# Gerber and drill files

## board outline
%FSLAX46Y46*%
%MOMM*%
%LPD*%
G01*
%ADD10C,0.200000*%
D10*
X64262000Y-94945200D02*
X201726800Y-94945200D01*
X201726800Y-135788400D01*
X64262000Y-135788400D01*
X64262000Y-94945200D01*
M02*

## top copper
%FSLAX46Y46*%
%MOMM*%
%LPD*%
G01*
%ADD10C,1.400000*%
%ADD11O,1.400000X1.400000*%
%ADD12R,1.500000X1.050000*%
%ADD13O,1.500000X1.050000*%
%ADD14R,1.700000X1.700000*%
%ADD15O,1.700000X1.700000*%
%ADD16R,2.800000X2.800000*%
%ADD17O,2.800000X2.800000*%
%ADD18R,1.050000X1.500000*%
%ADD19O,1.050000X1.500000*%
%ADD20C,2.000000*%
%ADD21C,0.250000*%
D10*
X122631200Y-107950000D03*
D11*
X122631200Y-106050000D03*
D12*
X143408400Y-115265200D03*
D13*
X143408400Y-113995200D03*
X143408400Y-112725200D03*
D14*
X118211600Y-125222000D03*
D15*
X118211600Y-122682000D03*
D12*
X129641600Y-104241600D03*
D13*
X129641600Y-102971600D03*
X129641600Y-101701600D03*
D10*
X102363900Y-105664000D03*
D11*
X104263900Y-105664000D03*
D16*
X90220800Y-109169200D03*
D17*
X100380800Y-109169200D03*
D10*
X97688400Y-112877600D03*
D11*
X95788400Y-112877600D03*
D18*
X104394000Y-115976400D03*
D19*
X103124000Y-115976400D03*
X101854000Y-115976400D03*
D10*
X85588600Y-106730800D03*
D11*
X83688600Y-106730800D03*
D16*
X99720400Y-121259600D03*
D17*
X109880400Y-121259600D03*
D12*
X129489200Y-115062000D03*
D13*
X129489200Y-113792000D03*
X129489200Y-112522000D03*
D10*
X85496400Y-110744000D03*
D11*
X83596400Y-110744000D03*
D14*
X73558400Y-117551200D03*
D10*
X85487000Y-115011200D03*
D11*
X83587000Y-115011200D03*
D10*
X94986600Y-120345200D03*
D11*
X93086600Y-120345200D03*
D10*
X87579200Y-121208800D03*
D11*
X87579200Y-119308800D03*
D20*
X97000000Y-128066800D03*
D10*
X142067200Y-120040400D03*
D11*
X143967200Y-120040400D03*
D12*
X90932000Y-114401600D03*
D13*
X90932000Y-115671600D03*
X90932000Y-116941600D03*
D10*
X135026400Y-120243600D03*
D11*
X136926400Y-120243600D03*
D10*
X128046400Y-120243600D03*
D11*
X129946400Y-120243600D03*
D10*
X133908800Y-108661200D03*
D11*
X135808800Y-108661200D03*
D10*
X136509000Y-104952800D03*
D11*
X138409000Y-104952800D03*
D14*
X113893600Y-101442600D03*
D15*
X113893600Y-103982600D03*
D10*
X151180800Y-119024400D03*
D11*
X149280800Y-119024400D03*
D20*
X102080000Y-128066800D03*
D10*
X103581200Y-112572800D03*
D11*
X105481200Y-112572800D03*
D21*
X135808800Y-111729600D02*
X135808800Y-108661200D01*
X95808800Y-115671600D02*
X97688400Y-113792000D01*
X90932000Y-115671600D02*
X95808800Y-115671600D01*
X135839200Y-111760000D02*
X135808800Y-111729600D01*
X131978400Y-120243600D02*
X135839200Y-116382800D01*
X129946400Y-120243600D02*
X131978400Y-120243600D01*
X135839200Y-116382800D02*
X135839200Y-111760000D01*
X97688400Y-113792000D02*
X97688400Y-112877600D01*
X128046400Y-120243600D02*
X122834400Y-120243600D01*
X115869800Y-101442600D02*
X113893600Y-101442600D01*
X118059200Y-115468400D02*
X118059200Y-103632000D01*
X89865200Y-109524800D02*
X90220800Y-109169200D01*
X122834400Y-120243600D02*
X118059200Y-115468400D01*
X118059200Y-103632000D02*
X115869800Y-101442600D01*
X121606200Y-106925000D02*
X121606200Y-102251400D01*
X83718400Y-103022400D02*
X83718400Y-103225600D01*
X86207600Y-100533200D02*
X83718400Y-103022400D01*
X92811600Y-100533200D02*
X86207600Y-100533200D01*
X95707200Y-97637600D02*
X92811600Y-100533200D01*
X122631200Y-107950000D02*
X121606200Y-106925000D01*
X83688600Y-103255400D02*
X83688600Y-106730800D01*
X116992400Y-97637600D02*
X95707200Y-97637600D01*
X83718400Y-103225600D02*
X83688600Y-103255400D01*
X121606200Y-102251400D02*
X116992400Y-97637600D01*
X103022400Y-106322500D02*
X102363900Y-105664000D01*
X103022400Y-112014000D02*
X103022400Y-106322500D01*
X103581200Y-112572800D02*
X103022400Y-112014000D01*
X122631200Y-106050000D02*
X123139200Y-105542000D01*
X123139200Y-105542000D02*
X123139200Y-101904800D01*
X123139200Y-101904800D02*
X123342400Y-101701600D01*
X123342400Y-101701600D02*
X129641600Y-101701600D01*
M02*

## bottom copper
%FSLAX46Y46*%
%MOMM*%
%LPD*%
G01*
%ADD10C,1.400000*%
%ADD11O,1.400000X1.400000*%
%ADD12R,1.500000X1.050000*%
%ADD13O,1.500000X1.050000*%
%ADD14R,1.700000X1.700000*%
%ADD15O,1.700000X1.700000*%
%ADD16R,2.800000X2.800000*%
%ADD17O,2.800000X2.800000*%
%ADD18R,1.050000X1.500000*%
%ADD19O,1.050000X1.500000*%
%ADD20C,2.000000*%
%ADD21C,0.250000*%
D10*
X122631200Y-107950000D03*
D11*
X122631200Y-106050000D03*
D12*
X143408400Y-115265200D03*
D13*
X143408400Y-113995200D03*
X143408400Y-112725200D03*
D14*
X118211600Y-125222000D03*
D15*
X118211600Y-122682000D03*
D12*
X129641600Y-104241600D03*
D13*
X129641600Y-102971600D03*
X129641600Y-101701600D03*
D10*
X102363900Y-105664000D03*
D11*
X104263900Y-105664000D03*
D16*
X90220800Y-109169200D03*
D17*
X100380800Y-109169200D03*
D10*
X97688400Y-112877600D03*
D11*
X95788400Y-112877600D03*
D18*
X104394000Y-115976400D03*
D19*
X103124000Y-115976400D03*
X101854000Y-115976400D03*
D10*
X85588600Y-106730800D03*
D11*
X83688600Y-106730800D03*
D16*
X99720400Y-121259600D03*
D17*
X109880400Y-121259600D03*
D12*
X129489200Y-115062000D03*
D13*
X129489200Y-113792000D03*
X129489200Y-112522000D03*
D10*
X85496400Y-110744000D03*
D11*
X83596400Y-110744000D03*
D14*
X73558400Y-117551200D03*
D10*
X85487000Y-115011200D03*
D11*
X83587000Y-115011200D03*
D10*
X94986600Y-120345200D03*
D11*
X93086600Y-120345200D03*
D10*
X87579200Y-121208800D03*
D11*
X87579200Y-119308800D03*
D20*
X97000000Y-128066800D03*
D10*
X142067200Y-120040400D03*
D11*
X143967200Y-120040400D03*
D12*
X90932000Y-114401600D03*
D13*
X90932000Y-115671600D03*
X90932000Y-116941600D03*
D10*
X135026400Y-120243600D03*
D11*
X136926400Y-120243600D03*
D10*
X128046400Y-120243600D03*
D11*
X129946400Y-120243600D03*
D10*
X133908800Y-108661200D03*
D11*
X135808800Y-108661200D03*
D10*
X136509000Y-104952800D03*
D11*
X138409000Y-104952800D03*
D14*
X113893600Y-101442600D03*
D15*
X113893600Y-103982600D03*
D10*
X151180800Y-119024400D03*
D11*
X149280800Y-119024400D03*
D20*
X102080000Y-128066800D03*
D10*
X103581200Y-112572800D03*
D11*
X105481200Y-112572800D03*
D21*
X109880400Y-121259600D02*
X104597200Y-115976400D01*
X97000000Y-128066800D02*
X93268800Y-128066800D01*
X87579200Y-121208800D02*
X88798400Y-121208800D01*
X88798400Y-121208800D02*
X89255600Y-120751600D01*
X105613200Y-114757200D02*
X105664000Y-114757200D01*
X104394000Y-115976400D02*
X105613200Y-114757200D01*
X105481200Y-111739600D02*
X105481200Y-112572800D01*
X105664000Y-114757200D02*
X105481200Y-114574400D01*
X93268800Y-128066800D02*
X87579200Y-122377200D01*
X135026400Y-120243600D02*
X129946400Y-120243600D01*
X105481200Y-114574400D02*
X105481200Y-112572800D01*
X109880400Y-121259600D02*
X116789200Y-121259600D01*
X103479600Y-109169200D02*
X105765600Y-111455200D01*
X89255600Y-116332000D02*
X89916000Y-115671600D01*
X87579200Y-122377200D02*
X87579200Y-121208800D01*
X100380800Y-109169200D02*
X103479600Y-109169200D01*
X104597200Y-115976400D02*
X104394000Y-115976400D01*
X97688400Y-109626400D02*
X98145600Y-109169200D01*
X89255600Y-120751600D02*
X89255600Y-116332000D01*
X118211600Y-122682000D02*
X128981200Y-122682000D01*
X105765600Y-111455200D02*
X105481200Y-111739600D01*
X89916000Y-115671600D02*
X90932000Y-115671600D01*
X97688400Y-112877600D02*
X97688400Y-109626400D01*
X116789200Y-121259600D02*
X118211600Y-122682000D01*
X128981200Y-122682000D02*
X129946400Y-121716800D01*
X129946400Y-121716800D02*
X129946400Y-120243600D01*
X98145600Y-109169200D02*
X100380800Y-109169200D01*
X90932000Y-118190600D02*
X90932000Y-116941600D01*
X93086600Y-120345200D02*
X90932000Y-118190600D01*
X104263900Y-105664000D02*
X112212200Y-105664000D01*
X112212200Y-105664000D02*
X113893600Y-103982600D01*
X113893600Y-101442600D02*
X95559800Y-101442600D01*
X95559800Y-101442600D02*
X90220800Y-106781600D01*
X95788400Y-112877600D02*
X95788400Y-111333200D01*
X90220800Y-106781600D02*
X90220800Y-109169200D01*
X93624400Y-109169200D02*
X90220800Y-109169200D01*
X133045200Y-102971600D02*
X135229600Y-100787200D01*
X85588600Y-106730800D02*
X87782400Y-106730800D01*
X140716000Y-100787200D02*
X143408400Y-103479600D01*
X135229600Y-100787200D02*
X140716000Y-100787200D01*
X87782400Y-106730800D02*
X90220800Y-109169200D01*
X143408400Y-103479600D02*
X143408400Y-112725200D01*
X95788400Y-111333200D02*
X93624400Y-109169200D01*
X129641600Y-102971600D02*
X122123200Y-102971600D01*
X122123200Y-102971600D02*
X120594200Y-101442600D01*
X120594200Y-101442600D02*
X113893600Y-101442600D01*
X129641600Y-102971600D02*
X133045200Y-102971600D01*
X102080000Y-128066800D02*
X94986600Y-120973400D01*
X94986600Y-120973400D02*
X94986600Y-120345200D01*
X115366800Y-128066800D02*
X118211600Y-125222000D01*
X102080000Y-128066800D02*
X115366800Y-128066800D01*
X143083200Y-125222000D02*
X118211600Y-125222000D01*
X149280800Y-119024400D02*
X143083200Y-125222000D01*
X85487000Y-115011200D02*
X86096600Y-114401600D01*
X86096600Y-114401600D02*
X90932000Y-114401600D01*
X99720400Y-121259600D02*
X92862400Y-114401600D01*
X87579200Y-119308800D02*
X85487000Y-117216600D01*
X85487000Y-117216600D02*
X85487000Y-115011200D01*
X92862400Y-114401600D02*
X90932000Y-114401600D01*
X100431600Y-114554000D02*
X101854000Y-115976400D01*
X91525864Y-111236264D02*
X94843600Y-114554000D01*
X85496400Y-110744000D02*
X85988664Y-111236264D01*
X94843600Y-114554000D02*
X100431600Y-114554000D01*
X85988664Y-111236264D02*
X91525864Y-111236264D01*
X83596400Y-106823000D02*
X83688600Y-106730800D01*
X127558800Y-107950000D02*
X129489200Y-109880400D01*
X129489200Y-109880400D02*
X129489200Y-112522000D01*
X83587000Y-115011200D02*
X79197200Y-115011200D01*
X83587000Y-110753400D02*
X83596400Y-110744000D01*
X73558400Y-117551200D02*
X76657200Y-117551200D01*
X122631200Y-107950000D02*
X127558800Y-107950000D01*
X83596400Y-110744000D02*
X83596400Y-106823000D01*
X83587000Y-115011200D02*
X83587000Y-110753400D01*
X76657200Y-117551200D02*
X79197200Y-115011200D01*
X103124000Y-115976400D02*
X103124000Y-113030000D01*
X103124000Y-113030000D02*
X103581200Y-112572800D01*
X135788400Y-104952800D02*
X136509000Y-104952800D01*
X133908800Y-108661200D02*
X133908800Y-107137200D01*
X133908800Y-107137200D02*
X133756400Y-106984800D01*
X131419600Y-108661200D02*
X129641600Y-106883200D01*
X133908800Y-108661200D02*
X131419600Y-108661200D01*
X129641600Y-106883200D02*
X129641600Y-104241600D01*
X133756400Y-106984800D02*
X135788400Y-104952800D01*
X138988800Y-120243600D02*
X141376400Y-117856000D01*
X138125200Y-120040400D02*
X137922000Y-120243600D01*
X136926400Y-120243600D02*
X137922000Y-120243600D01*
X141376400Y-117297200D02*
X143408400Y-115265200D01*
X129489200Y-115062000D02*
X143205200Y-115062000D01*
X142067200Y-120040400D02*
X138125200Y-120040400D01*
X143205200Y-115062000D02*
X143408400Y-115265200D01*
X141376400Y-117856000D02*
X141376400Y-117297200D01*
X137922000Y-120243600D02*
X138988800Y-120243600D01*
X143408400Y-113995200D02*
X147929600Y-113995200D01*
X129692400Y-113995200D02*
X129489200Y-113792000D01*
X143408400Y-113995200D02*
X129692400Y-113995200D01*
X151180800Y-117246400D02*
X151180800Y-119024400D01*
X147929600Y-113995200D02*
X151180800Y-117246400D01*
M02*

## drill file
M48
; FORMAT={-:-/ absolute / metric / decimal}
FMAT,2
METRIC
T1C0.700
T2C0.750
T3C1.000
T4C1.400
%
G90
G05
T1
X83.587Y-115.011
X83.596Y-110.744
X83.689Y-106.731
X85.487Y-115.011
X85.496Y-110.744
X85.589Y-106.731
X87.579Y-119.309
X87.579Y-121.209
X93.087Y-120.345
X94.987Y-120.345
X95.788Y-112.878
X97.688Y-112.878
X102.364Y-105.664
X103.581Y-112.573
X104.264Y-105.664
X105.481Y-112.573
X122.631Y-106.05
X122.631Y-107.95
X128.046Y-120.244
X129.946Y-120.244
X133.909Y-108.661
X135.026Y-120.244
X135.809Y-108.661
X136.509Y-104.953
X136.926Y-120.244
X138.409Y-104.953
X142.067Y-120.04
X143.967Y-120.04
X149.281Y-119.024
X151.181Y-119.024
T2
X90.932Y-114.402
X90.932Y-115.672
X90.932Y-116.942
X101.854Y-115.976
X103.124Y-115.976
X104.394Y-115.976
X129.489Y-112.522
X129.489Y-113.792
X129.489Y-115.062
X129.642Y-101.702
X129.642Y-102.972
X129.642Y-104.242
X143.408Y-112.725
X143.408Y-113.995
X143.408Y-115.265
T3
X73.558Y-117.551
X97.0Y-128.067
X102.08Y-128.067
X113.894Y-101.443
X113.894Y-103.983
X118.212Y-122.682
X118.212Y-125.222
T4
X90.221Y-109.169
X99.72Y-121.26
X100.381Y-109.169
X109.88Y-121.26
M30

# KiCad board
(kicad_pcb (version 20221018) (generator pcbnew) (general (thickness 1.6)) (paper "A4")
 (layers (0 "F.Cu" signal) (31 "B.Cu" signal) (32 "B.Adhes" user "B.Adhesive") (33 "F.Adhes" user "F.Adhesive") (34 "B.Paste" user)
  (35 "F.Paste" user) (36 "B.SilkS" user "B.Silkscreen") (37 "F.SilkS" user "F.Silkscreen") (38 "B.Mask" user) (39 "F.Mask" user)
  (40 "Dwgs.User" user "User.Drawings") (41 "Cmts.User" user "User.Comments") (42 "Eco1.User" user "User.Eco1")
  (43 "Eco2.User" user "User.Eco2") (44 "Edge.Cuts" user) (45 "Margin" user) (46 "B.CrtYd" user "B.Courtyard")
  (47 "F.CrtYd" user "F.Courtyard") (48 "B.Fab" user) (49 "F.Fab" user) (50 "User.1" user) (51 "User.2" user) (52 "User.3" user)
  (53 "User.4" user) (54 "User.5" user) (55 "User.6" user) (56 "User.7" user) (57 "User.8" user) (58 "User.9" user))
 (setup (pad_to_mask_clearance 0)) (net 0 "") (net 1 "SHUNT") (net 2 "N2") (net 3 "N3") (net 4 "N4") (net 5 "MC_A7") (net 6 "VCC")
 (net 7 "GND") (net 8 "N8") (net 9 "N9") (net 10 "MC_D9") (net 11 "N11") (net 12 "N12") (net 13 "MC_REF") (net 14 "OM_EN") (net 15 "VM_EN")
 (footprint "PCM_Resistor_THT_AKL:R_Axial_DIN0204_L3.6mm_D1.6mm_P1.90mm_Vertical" (layer "F.Cu") (at 122.6312 107.95 90)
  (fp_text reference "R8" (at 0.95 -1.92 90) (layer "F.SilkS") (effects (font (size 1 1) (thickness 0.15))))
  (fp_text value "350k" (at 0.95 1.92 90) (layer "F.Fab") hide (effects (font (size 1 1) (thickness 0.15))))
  (pad "1" thru_hole circle (at 0 0 90) (size 1.4 1.4) (drill 0.7) (layers "*.Cu" "*.Mask") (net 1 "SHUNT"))
  (pad "2" thru_hole oval (at 1.9 0 90) (size 1.4 1.4) (drill 0.7) (layers "*.Cu" "*.Mask") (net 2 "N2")))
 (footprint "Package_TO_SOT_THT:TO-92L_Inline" (layer "F.Cu") (at 143.4084 115.2652 90)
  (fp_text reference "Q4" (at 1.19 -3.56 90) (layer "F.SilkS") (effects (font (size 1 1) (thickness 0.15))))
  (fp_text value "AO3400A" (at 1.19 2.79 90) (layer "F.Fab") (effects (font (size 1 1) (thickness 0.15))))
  (pad "1" thru_hole rect (at 0 0 90) (size 1.05 1.5) (drill 0.75) (layers "*.Cu" "*.Mask") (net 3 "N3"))
  (pad "2" thru_hole oval (at 1.27 0 90) (size 1.05 1.5) (drill 0.75) (layers "*.Cu" "*.Mask") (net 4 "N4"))
  (pad "3" thru_hole oval (at 2.54 0 90) (size 1.05 1.5) (drill 0.75) (layers "*.Cu" "*.Mask") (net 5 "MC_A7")))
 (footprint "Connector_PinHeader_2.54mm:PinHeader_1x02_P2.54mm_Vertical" (layer "F.Cu") (at 118.2116 125.222 180)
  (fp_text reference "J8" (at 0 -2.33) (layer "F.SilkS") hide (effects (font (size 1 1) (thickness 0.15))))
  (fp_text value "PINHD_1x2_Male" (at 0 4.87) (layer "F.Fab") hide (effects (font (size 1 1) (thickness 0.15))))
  (pad "1" thru_hole rect (at 0 0 180) (size 1.7 1.7) (drill 1) (layers "*.Cu" "*.Mask") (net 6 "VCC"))
  (pad "2" thru_hole oval (at 0 2.54 180) (size 1.7 1.7) (drill 1) (layers "*.Cu" "*.Mask") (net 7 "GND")))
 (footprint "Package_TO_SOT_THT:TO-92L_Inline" (layer "F.Cu") (at 129.6416 104.2416 90)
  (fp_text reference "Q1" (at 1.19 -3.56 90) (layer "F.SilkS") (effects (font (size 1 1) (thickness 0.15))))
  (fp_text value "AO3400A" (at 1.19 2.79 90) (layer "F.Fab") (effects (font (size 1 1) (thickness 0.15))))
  (pad "1" thru_hole rect (at 0 0 90) (size 1.05 1.5) (drill 0.75) (layers "*.Cu" "*.Mask") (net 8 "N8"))
  (pad "2" thru_hole oval (at 1.27 0 90) (size 1.05 1.5) (drill 0.75) (layers "*.Cu" "*.Mask") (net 5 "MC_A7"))
  (pad "3" thru_hole oval (at 2.54 0 90) (size 1.05 1.5) (drill 0.75) (layers "*.Cu" "*.Mask") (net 2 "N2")))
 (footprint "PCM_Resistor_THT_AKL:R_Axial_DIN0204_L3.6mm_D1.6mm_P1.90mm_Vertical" (layer "F.Cu") (at 102.3639 105.664)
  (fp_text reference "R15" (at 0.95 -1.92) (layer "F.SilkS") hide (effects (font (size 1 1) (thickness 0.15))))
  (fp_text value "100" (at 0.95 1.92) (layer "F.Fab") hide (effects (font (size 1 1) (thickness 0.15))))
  (pad "1" thru_hole circle (at 0 0) (size 1.4 1.4) (drill 0.7) (layers "*.Cu" "*.Mask") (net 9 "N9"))
  (pad "2" thru_hole oval (at 1.9 0) (size 1.4 1.4) (drill 0.7) (layers "*.Cu" "*.Mask") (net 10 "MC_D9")))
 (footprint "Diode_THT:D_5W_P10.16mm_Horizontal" (layer "F.Cu") (at 90.2208 109.1692)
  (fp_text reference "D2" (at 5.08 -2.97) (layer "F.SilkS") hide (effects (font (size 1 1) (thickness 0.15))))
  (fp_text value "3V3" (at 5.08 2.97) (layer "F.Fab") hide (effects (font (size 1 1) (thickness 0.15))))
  (pad "1" thru_hole rect (at 0 0) (size 2.8 2.8) (drill 1.4) (layers "*.Cu" "*.Mask") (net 5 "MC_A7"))
  (pad "2" thru_hole oval (at 10.16 0) (size 2.8 2.8) (drill 1.4) (layers "*.Cu" "*.Mask") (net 7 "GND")))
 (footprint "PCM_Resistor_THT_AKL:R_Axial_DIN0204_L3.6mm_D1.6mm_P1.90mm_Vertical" (layer "F.Cu") (at 97.6884 112.8776 180)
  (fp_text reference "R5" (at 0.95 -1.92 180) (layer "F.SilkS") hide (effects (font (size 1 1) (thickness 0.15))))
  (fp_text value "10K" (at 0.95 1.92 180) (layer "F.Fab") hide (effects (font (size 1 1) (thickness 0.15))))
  (pad "1" thru_hole circle (at 0 0 180) (size 1.4 1.4) (drill 0.7) (layers "*.Cu" "*.Mask") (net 7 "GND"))
  (pad "2" thru_hole oval (at 1.9 0 180) (size 1.4 1.4) (drill 0.7) (layers "*.Cu" "*.Mask") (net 5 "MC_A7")))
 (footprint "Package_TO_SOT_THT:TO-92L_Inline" (layer "F.Cu") (at 104.394 115.9764 180)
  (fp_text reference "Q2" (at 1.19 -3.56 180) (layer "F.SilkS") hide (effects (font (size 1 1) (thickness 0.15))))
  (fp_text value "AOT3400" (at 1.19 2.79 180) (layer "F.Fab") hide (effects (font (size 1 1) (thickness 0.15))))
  (pad "1" thru_hole rect (at 0 0 180) (size 1.05 1.5) (drill 0.75) (layers "*.Cu" "*.Mask") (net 7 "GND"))
  (pad "2" thru_hole oval (at 1.27 0 180) (size 1.05 1.5) (drill 0.75) (layers "*.Cu" "*.Mask") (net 9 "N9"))
  (pad "3" thru_hole oval (at 2.54 0 180) (size 1.05 1.5) (drill 0.75) (layers "*.Cu" "*.Mask") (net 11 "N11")))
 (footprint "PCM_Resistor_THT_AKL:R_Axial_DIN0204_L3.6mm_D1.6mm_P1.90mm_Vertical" (layer "F.Cu") (at 85.5886 106.7308 180)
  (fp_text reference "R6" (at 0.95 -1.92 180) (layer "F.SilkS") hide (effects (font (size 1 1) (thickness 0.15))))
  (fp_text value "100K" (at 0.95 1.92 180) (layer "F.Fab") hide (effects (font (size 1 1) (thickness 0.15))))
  (pad "1" thru_hole circle (at 0 0 180) (size 1.4 1.4) (drill 0.7) (layers "*.Cu" "*.Mask") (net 5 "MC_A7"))
  (pad "2" thru_hole oval (at 1.9 0 180) (size 1.4 1.4) (drill 0.7) (layers "*.Cu" "*.Mask") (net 1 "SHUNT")))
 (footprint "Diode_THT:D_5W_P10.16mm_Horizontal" (layer "F.Cu") (at 99.7204 121.2596)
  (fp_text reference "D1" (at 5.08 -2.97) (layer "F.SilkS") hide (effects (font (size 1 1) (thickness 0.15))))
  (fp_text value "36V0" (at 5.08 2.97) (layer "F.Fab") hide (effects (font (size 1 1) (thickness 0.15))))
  (pad "1" thru_hole rect (at 0 0) (size 2.8 2.8) (drill 1.4) (layers "*.Cu" "*.Mask") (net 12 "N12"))
  (pad "2" thru_hole oval (at 10.16 0) (size 2.8 2.8) (drill 1.4) (layers "*.Cu" "*.Mask") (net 7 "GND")))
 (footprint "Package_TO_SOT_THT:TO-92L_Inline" (layer "F.Cu") (at 129.4892 115.062 90)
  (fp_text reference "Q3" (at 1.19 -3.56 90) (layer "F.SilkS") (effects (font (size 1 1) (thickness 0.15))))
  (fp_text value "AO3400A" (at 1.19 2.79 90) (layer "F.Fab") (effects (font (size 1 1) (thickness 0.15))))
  (pad "1" thru_hole rect (at 0 0 90) (size 1.05 1.5) (drill 0.75) (layers "*.Cu" "*.Mask") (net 3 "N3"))
  (pad "2" thru_hole oval (at 1.27 0 90) (size 1.05 1.5) (drill 0.75) (layers "*.Cu" "*.Mask") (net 4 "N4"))
  (pad "3" thru_hole oval (at 2.54 0 90) (size 1.05 1.5) (drill 0.75) (layers "*.Cu" "*.Mask") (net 1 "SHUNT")))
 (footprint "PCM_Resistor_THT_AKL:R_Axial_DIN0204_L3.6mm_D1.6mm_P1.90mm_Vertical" (layer "F.Cu") (at 85.4964 110.744 180)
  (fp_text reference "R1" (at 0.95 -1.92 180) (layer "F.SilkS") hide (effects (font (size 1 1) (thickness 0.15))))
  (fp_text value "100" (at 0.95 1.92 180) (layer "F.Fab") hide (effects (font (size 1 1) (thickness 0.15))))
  (pad "1" thru_hole circle (at 0 0 180) (size 1.4 1.4) (drill 0.7) (layers "*.Cu" "*.Mask") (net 11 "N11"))
  (pad "2" thru_hole oval (at 1.9 0 180) (size 1.4 1.4) (drill 0.7) (layers "*.Cu" "*.Mask") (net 1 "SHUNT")))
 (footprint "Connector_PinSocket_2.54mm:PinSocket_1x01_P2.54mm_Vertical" (layer "F.Cu") (at 73.5584 117.5512)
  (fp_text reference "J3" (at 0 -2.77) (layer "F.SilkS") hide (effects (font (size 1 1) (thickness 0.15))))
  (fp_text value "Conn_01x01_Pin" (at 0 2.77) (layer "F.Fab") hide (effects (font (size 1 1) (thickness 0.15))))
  (pad "1" thru_hole rect (at 0 0) (size 1.7 1.7) (drill 1) (layers "*.Cu" "*.Mask") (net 1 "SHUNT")))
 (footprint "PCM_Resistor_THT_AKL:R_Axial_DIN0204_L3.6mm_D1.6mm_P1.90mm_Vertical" (layer "F.Cu") (at 85.487 115.0112 180)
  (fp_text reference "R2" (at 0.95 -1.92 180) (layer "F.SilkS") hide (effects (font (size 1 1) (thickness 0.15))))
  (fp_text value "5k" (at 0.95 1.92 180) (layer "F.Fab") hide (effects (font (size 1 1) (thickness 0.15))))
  (pad "1" thru_hole circle (at 0 0 180) (size 1.4 1.4) (drill 0.7) (layers "*.Cu" "*.Mask") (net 12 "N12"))
  (pad "2" thru_hole oval (at 1.9 0 180) (size 1.4 1.4) (drill 0.7) (layers "*.Cu" "*.Mask") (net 1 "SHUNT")))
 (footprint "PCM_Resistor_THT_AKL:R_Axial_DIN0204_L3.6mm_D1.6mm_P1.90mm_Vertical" (layer "F.Cu") (at 94.9866 120.3452 180)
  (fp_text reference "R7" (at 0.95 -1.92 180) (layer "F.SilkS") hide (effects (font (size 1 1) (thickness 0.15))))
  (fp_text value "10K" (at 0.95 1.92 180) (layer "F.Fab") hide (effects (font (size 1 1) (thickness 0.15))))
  (pad "1" thru_hole circle (at 0 0 180) (size 1.4 1.4) (drill 0.7) (layers "*.Cu" "*.Mask") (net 6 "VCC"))
  (pad "2" thru_hole oval (at 1.9 0 180) (size 1.4 1.4) (drill 0.7) (layers "*.Cu" "*.Mask") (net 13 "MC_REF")))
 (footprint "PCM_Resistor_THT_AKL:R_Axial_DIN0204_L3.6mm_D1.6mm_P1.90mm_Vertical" (layer "F.Cu") (at 87.5792 121.2088 90)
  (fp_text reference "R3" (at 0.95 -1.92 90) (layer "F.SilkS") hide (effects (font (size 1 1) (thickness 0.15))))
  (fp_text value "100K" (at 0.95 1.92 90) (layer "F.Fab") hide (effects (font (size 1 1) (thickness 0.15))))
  (pad "1" thru_hole circle (at 0 0 90) (size 1.4 1.4) (drill 0.7) (layers "*.Cu" "*.Mask") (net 7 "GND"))
  (pad "2" thru_hole oval (at 1.9 0 90) (size 1.4 1.4) (drill 0.7) (layers "*.Cu" "*.Mask") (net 12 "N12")))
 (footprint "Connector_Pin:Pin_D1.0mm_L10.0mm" (layer "F.Cu") (at 97 128.0668 180)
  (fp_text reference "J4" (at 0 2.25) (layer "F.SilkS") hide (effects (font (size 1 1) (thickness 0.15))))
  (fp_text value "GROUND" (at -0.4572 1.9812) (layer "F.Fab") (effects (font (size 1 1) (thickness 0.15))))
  (pad "1" thru_hole circle (at 0 0 180) (size 2 2) (drill 1) (layers "*.Cu" "*.Mask") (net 7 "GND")))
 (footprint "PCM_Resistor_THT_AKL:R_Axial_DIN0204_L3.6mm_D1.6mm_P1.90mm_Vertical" (layer "F.Cu") (at 142.0672 120.0404)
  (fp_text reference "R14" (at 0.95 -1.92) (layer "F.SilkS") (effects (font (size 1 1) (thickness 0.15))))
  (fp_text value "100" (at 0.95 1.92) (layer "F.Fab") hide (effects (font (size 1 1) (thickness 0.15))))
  (pad "1" thru_hole circle (at 0 0) (size 1.4 1.4) (drill 0.7) (layers "*.Cu" "*.Mask") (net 3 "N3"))
  (pad "2" thru_hole oval (at 1.9 0) (size 1.4 1.4) (drill 0.7) (layers "*.Cu" "*.Mask") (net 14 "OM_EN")))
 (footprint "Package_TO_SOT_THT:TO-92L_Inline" (layer "F.Cu") (at 90.932 114.4016 -90)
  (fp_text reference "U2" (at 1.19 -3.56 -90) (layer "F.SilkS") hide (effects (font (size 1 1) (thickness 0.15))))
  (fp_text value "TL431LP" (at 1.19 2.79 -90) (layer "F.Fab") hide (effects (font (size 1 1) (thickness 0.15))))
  (pad "1" thru_hole rect (at 0 0 270) (size 1.05 1.5) (drill 0.75) (layers "*.Cu" "*.Mask") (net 12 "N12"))
  (pad "2" thru_hole oval (at 1.27 0 270) (size 1.05 1.5) (drill 0.75) (layers "*.Cu" "*.Mask") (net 7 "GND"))
  (pad "3" thru_hole oval (at 2.54 0 270) (size 1.05 1.5) (drill 0.75) (layers "*.Cu" "*.Mask") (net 13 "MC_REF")))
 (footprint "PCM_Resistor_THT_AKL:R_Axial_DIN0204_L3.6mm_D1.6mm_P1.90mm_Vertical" (layer "F.Cu") (at 135.0264 120.2436)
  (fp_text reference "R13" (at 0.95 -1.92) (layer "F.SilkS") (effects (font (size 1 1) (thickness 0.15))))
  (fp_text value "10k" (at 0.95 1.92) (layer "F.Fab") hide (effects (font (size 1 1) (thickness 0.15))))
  (pad "1" thru_hole circle (at 0 0) (size 1.4 1.4) (drill 0.7) (layers "*.Cu" "*.Mask") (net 7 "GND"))
  (pad "2" thru_hole oval (at 1.9 0) (size 1.4 1.4) (drill 0.7) (layers "*.Cu" "*.Mask") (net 3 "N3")))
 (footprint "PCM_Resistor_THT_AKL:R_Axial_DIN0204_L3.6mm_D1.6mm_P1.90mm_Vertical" (layer "F.Cu") (at 128.0464 120.2436)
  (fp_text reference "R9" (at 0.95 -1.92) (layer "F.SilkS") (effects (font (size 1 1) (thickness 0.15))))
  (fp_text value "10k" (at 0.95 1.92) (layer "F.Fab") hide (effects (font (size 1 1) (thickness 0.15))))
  (pad "1" thru_hole circle (at 0 0) (size 1.4 1.4) (drill 0.7) (layers "*.Cu" "*.Mask") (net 5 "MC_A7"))
  (pad "2" thru_hole oval (at 1.9 0) (size 1.4 1.4) (drill 0.7) (layers "*.Cu" "*.Mask") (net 7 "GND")))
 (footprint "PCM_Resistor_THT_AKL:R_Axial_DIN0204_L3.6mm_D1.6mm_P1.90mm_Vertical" (layer "F.Cu") (at 133.9088 108.6612)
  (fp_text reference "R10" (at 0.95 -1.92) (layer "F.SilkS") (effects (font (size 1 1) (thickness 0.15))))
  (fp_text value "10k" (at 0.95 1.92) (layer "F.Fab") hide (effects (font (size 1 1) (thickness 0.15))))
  (pad "1" thru_hole circle (at 0 0) (size 1.4 1.4) (drill 0.7) (layers "*.Cu" "*.Mask") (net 8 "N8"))
  (pad "2" thru_hole oval (at 1.9 0) (size 1.4 1.4) (drill 0.7) (layers "*.Cu" "*.Mask") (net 7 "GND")))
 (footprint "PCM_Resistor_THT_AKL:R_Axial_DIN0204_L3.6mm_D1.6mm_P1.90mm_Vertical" (layer "F.Cu") (at 136.509 104.9528)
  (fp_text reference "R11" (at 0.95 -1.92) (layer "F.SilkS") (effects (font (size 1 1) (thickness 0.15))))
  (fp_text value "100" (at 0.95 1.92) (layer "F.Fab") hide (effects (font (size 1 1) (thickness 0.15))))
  (pad "1" thru_hole circle (at 0 0) (size 1.4 1.4) (drill 0.7) (layers "*.Cu" "*.Mask") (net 8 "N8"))
  (pad "2" thru_hole oval (at 1.9 0) (size 1.4 1.4) (drill 0.7) (layers "*.Cu" "*.Mask") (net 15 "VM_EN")))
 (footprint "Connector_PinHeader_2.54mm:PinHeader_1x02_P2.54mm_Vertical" (layer "F.Cu") (at 113.8936 101.4426)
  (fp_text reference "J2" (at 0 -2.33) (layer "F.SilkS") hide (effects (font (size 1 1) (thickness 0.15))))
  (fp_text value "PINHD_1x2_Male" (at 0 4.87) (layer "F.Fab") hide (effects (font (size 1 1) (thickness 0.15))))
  (pad "1" thru_hole rect (at 0 0) (size 1.7 1.7) (drill 1) (layers "*.Cu" "*.Mask") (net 5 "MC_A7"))
  (pad "2" thru_hole oval (at 0 2.54) (size 1.7 1.7) (drill 1) (layers "*.Cu" "*.Mask") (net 10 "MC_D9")))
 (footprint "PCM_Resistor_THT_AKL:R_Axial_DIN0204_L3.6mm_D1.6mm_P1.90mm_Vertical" (layer "F.Cu") (at 151.1808 119.0244 180)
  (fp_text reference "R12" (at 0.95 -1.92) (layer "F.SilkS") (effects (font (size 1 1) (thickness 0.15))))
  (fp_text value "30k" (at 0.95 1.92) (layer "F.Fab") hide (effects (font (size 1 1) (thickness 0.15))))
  (pad "1" thru_hole circle (at 0 0 180) (size 1.4 1.4) (drill 0.7) (layers "*.Cu" "*.Mask") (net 4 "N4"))
  (pad "2" thru_hole oval (at 1.9 0 180) (size 1.4 1.4) (drill 0.7) (layers "*.Cu" "*.Mask") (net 6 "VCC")))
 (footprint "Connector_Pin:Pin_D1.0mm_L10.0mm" (layer "F.Cu") (at 102.08 128.0668)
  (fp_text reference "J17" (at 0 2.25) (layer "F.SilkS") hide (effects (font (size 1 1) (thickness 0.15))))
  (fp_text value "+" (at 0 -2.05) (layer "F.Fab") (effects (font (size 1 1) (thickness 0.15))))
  (pad "1" thru_hole circle (at 0 0) (size 2 2) (drill 1) (layers "*.Cu" "*.Mask") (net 6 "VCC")))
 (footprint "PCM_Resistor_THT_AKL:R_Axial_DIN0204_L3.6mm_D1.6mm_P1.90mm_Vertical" (layer "F.Cu") (at 103.5812 112.5728)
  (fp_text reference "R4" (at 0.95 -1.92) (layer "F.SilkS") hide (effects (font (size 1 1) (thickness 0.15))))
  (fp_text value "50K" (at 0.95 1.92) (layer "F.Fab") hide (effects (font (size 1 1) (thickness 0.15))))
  (pad "1" thru_hole circle (at 0 0) (size 1.4 1.4) (drill 0.7) (layers "*.Cu" "*.Mask") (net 9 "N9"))
  (pad "2" thru_hole oval (at 1.9 0) (size 1.4 1.4) (drill 0.7) (layers "*.Cu" "*.Mask") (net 7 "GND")))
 (gr_rect (start 64.262 94.9452) (end 201.7268 135.7884) (stroke (width 0.2) (type default)) (fill none) (layer "Edge.Cuts"))
 (segment (start 135.8088 111.7296) (end 135.8088 108.6612) (width 0.25) (layer "F.Cu") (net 7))
 (segment (start 95.8088 115.6716) (end 97.6884 113.792) (width 0.25) (layer "F.Cu") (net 7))
 (segment (start 90.932 115.6716) (end 95.8088 115.6716) (width 0.25) (layer "F.Cu") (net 7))
 (segment (start 135.8392 111.76) (end 135.8088 111.7296) (width 0.25) (layer "F.Cu") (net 7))
 (segment (start 131.9784 120.2436) (end 135.8392 116.3828) (width 0.25) (layer "F.Cu") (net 7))
 (segment (start 129.9464 120.2436) (end 131.9784 120.2436) (width 0.25) (layer "F.Cu") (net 7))
 (segment (start 135.8392 116.3828) (end 135.8392 111.76) (width 0.25) (layer "F.Cu") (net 7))
 (segment (start 97.6884 113.792) (end 97.6884 112.8776) (width 0.25) (layer "F.Cu") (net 7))
 (segment (start 109.8804 121.2596) (end 104.5972 115.9764) (width 0.25) (layer "B.Cu") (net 7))
 (segment (start 97 128.0668) (end 93.2688 128.0668) (width 0.25) (layer "B.Cu") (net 7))
 (segment (start 87.5792 121.2088) (end 88.7984 121.2088) (width 0.25) (layer "B.Cu") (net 7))
 (segment (start 88.7984 121.2088) (end 89.2556 120.7516) (width 0.25) (layer "B.Cu") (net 7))
 (segment (start 105.6132 114.7572) (end 105.664 114.7572) (width 0.25) (layer "B.Cu") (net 7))
 (segment (start 104.394 115.9764) (end 105.6132 114.7572) (width 0.25) (layer "B.Cu") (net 7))
 (segment (start 105.4812 111.7396) (end 105.4812 112.5728) (width 0.25) (layer "B.Cu") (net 7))
 (segment (start 105.664 114.7572) (end 105.4812 114.5744) (width 0.25) (layer "B.Cu") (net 7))
 (segment (start 93.2688 128.0668) (end 87.5792 122.3772) (width 0.25) (layer "B.Cu") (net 7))
 (segment (start 135.0264 120.2436) (end 129.9464 120.2436) (width 0.25) (layer "B.Cu") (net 7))
 (segment (start 105.4812 114.5744) (end 105.4812 112.5728) (width 0.25) (layer "B.Cu") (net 7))
 (segment (start 109.8804 121.2596) (end 116.7892 121.2596) (width 0.25) (layer "B.Cu") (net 7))
 (segment (start 103.4796 109.1692) (end 105.7656 111.4552) (width 0.25) (layer "B.Cu") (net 7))
 (segment (start 89.2556 116.332) (end 89.916 115.6716) (width 0.25) (layer "B.Cu") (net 7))
 (segment (start 87.5792 122.3772) (end 87.5792 121.2088) (width 0.25) (layer "B.Cu") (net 7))
 (segment (start 100.3808 109.1692) (end 103.4796 109.1692) (width 0.25) (layer "B.Cu") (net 7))
 (segment (start 104.5972 115.9764) (end 104.394 115.9764) (width 0.25) (layer "B.Cu") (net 7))
 (segment (start 97.6884 109.6264) (end 98.1456 109.1692) (width 0.25) (layer "B.Cu") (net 7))
 (segment (start 89.2556 120.7516) (end 89.2556 116.332) (width 0.25) (layer "B.Cu") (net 7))
 (segment (start 118.2116 122.682) (end 128.9812 122.682) (width 0.25) (layer "B.Cu") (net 7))
 (segment (start 105.7656 111.4552) (end 105.4812 111.7396) (width 0.25) (layer "B.Cu") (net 7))
 (segment (start 89.916 115.6716) (end 90.932 115.6716) (width 0.25) (layer "B.Cu") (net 7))
 (segment (start 97.6884 112.8776) (end 97.6884 109.6264) (width 0.25) (layer "B.Cu") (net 7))
 (segment (start 116.7892 121.2596) (end 118.2116 122.682) (width 0.25) (layer "B.Cu") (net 7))
 (segment (start 128.9812 122.682) (end 129.9464 121.7168) (width 0.25) (layer "B.Cu") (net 7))
 (segment (start 129.9464 121.7168) (end 129.9464 120.2436) (width 0.25) (layer "B.Cu") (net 7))
 (segment (start 98.1456 109.1692) (end 100.3808 109.1692) (width 0.25) (layer "B.Cu") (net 7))
 (segment (start 90.932 118.1906) (end 90.932 116.9416) (width 0.25) (layer "B.Cu") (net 13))
 (segment (start 93.0866 120.3452) (end 90.932 118.1906) (width 0.25) (layer "B.Cu") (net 13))
 (segment (start 104.2639 105.664) (end 112.2122 105.664) (width 0.25) (layer "B.Cu") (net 10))
 (segment (start 112.2122 105.664) (end 113.8936 103.9826) (width 0.25) (layer "B.Cu") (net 10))
 (segment (start 128.0464 120.2436) (end 122.8344 120.2436) (width 0.25) (layer "F.Cu") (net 5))
 (segment (start 115.8698 101.4426) (end 113.8936 101.4426) (width 0.25) (layer "F.Cu") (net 5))
 (segment (start 118.0592 115.4684) (end 118.0592 103.632) (width 0.25) (layer "F.Cu") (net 5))
 (segment (start 89.8652 109.5248) (end 90.2208 109.1692) (width 0.25) (layer "F.Cu") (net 5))
 (segment (start 122.8344 120.2436) (end 118.0592 115.4684) (width 0.25) (layer "F.Cu") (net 5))
 (segment (start 118.0592 103.632) (end 115.8698 101.4426) (width 0.25) (layer "F.Cu") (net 5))
 (segment (start 113.8936 101.4426) (end 95.5598 101.4426) (width 0.25) (layer "B.Cu") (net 5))
 (segment (start 95.5598 101.4426) (end 90.2208 106.7816) (width 0.25) (layer "B.Cu") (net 5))
 (segment (start 95.7884 112.8776) (end 95.7884 111.3332) (width 0.25) (layer "B.Cu") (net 5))
 (segment (start 90.2208 106.7816) (end 90.2208 109.1692) (width 0.25) (layer "B.Cu") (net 5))
 (segment (start 93.6244 109.1692) (end 90.2208 109.1692) (width 0.25) (layer "B.Cu") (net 5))
 (segment (start 133.0452 102.9716) (end 135.2296 100.7872) (width 0.25) (layer "B.Cu") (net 5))
 (segment (start 85.5886 106.7308) (end 87.7824 106.7308) (width 0.25) (layer "B.Cu") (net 5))
 (segment (start 140.716 100.7872) (end 143.4084 103.4796) (width 0.25) (layer "B.Cu") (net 5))
 (segment (start 135.2296 100.7872) (end 140.716 100.7872) (width 0.25) (layer "B.Cu") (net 5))
 (segment (start 87.7824 106.7308) (end 90.2208 109.1692) (width 0.25) (layer "B.Cu") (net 5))
 (segment (start 143.4084 103.4796) (end 143.4084 112.7252) (width 0.25) (layer "B.Cu") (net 5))
 (segment (start 95.7884 111.3332) (end 93.6244 109.1692) (width 0.25) (layer "B.Cu") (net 5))
 (segment (start 129.6416 102.9716) (end 122.1232 102.9716) (width 0.25) (layer "B.Cu") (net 5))
 (segment (start 122.1232 102.9716) (end 120.5942 101.4426) (width 0.25) (layer "B.Cu") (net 5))
 (segment (start 120.5942 101.4426) (end 113.8936 101.4426) (width 0.25) (layer "B.Cu") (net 5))
 (segment (start 129.6416 102.9716) (end 133.0452 102.9716) (width 0.25) (layer "B.Cu") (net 5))
 (segment (start 102.08 128.0668) (end 94.9866 120.9734) (width 0.25) (layer "B.Cu") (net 6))
 (segment (start 94.9866 120.9734) (end 94.9866 120.3452) (width 0.25) (layer "B.Cu") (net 6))
 (segment (start 115.3668 128.0668) (end 118.2116 125.222) (width 0.25) (layer "B.Cu") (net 6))
 (segment (start 102.08 128.0668) (end 115.3668 128.0668) (width 0.25) (layer "B.Cu") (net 6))
 (segment (start 143.0832 125.222) (end 118.2116 125.222) (width 0.25) (layer "B.Cu") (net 6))
 (segment (start 149.2808 119.0244) (end 143.0832 125.222) (width 0.25) (layer "B.Cu") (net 6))
 (segment (start 85.487 115.0112) (end 86.0966 114.4016) (width 0.25) (layer "B.Cu") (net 12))
 (segment (start 86.0966 114.4016) (end 90.932 114.4016) (width 0.25) (layer "B.Cu") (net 12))
 (segment (start 99.7204 121.2596) (end 92.8624 114.4016) (width 0.25) (layer "B.Cu") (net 12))
 (segment (start 87.5792 119.3088) (end 85.487 117.2166) (width 0.25) (layer "B.Cu") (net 12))
 (segment (start 85.487 117.2166) (end 85.487 115.0112) (width 0.25) (layer "B.Cu") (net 12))
 (segment (start 92.8624 114.4016) (end 90.932 114.4016) (width 0.25) (layer "B.Cu") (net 12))
 (segment (start 100.4316 114.554) (end 101.854 115.9764) (width 0.25) (layer "B.Cu") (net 11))
 (segment (start 91.525864 111.236264) (end 94.8436 114.554) (width 0.25) (layer "B.Cu") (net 11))
 (segment (start 85.4964 110.744) (end 85.988664 111.236264) (width 0.25) (layer "B.Cu") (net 11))
 (segment (start 94.8436 114.554) (end 100.4316 114.554) (width 0.25) (layer "B.Cu") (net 11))
 (segment (start 85.988664 111.236264) (end 91.525864 111.236264) (width 0.25) (layer "B.Cu") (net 11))
 (segment (start 121.6062 106.925) (end 121.6062 102.2514) (width 0.25) (layer "F.Cu") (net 1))
 (segment (start 83.7184 103.0224) (end 83.7184 103.2256) (width 0.25) (layer "F.Cu") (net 1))
 (segment (start 86.2076 100.5332) (end 83.7184 103.0224) (width 0.25) (layer "F.Cu") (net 1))
 (segment (start 92.8116 100.5332) (end 86.2076 100.5332) (width 0.25) (layer "F.Cu") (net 1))
 (segment (start 95.7072 97.6376) (end 92.8116 100.5332) (width 0.25) (layer "F.Cu") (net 1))
 (segment (start 122.6312 107.95) (end 121.6062 106.925) (width 0.25) (layer "F.Cu") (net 1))
 (segment (start 83.6886 103.2554) (end 83.6886 106.7308) (width 0.25) (layer "F.Cu") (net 1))
 (segment (start 116.9924 97.6376) (end 95.7072 97.6376) (width 0.25) (layer "F.Cu") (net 1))
 (segment (start 83.7184 103.2256) (end 83.6886 103.2554) (width 0.25) (layer "F.Cu") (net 1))
 (segment (start 121.6062 102.2514) (end 116.9924 97.6376) (width 0.25) (layer "F.Cu") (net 1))
 (segment (start 83.5964 106.823) (end 83.6886 106.7308) (width 0.25) (layer "B.Cu") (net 1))
 (segment (start 127.5588 107.95) (end 129.4892 109.8804) (width 0.25) (layer "B.Cu") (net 1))
 (segment (start 129.4892 109.8804) (end 129.4892 112.522) (width 0.25) (layer "B.Cu") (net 1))
 (segment (start 83.587 115.0112) (end 79.1972 115.0112) (width 0.25) (layer "B.Cu") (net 1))
 (segment (start 83.587 110.7534) (end 83.5964 110.744) (width 0.25) (layer "B.Cu") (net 1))
 (segment (start 73.5584 117.5512) (end 76.6572 117.5512) (width 0.25) (layer "B.Cu") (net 1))
 (segment (start 122.6312 107.95) (end 127.5588 107.95) (width 0.25) (layer "B.Cu") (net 1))
 (segment (start 83.5964 110.744) (end 83.5964 106.823) (width 0.25) (layer "B.Cu") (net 1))
 (segment (start 83.587 115.0112) (end 83.587 110.7534) (width 0.25) (layer "B.Cu") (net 1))
 (segment (start 76.6572 117.5512) (end 79.1972 115.0112) (width 0.25) (layer "B.Cu") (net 1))
 (segment (start 103.0224 106.3225) (end 102.3639 105.664) (width 0.25) (layer "F.Cu") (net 9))
 (segment (start 103.0224 112.014) (end 103.0224 106.3225) (width 0.25) (layer "F.Cu") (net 9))
 (segment (start 103.5812 112.5728) (end 103.0224 112.014) (width 0.25) (layer "F.Cu") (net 9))
 (segment (start 103.124 115.9764) (end 103.124 113.03) (width 0.25) (layer "B.Cu") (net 9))
 (segment (start 103.124 113.03) (end 103.5812 112.5728) (width 0.25) (layer "B.Cu") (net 9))
 (segment (start 135.7884 104.9528) (end 136.509 104.9528) (width 0.25) (layer "B.Cu") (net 8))
 (segment (start 133.9088 108.6612) (end 133.9088 107.1372) (width 0.25) (layer "B.Cu") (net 8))
 (segment (start 133.9088 107.1372) (end 133.7564 106.9848) (width 0.25) (layer "B.Cu") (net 8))
 (segment (start 131.4196 108.6612) (end 129.6416 106.8832) (width 0.25) (layer "B.Cu") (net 8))
 (segment (start 133.9088 108.6612) (end 131.4196 108.6612) (width 0.25) (layer "B.Cu") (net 8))
 (segment (start 129.6416 106.8832) (end 129.6416 104.2416) (width 0.25) (layer "B.Cu") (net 8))
 (segment (start 133.7564 106.9848) (end 135.7884 104.9528) (width 0.25) (layer "B.Cu") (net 8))
 (segment (start 122.6312 106.05) (end 123.1392 105.542) (width 0.25) (layer "F.Cu") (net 2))
 (segment (start 123.1392 105.542) (end 123.1392 101.9048) (width 0.25) (layer "F.Cu") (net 2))
 (segment (start 123.1392 101.9048) (end 123.3424 101.7016) (width 0.25) (layer "F.Cu") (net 2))
 (segment (start 123.3424 101.7016) (end 129.6416 101.7016) (width 0.25) (layer "F.Cu") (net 2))
 (segment (start 138.9888 120.2436) (end 141.3764 117.856) (width 0.25) (layer "B.Cu") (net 3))
 (segment (start 138.1252 120.0404) (end 137.922 120.2436) (width 0.25) (layer "B.Cu") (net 3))
 (segment (start 136.9264 120.2436) (end 137.922 120.2436) (width 0.25) (layer "B.Cu") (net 3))
 (segment (start 141.3764 117.2972) (end 143.4084 115.2652) (width 0.25) (layer "B.Cu") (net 3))
 (segment (start 129.4892 115.062) (end 143.2052 115.062) (width 0.25) (layer "B.Cu") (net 3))
 (segment (start 142.0672 120.0404) (end 138.1252 120.0404) (width 0.25) (layer "B.Cu") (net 3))
 (segment (start 143.2052 115.062) (end 143.4084 115.2652) (width 0.25) (layer "B.Cu") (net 3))
 (segment (start 141.3764 117.856) (end 141.3764 117.2972) (width 0.25) (layer "B.Cu") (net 3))
 (segment (start 137.922 120.2436) (end 138.9888 120.2436) (width 0.25) (layer "B.Cu") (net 3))
 (segment (start 143.4084 113.9952) (end 147.9296 113.9952) (width 0.25) (layer "B.Cu") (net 4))
 (segment (start 129.6924 113.9952) (end 129.4892 113.792) (width 0.25) (layer "B.Cu") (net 4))
 (segment (start 143.4084 113.9952) (end 129.6924 113.9952) (width 0.25) (layer "B.Cu") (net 4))
 (segment (start 151.1808 117.2464) (end 151.1808 119.0244) (width 0.25) (layer "B.Cu") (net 4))
 (segment (start 147.9296 113.9952) (end 151.1808 117.2464) (width 0.25) (layer "B.Cu") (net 4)))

